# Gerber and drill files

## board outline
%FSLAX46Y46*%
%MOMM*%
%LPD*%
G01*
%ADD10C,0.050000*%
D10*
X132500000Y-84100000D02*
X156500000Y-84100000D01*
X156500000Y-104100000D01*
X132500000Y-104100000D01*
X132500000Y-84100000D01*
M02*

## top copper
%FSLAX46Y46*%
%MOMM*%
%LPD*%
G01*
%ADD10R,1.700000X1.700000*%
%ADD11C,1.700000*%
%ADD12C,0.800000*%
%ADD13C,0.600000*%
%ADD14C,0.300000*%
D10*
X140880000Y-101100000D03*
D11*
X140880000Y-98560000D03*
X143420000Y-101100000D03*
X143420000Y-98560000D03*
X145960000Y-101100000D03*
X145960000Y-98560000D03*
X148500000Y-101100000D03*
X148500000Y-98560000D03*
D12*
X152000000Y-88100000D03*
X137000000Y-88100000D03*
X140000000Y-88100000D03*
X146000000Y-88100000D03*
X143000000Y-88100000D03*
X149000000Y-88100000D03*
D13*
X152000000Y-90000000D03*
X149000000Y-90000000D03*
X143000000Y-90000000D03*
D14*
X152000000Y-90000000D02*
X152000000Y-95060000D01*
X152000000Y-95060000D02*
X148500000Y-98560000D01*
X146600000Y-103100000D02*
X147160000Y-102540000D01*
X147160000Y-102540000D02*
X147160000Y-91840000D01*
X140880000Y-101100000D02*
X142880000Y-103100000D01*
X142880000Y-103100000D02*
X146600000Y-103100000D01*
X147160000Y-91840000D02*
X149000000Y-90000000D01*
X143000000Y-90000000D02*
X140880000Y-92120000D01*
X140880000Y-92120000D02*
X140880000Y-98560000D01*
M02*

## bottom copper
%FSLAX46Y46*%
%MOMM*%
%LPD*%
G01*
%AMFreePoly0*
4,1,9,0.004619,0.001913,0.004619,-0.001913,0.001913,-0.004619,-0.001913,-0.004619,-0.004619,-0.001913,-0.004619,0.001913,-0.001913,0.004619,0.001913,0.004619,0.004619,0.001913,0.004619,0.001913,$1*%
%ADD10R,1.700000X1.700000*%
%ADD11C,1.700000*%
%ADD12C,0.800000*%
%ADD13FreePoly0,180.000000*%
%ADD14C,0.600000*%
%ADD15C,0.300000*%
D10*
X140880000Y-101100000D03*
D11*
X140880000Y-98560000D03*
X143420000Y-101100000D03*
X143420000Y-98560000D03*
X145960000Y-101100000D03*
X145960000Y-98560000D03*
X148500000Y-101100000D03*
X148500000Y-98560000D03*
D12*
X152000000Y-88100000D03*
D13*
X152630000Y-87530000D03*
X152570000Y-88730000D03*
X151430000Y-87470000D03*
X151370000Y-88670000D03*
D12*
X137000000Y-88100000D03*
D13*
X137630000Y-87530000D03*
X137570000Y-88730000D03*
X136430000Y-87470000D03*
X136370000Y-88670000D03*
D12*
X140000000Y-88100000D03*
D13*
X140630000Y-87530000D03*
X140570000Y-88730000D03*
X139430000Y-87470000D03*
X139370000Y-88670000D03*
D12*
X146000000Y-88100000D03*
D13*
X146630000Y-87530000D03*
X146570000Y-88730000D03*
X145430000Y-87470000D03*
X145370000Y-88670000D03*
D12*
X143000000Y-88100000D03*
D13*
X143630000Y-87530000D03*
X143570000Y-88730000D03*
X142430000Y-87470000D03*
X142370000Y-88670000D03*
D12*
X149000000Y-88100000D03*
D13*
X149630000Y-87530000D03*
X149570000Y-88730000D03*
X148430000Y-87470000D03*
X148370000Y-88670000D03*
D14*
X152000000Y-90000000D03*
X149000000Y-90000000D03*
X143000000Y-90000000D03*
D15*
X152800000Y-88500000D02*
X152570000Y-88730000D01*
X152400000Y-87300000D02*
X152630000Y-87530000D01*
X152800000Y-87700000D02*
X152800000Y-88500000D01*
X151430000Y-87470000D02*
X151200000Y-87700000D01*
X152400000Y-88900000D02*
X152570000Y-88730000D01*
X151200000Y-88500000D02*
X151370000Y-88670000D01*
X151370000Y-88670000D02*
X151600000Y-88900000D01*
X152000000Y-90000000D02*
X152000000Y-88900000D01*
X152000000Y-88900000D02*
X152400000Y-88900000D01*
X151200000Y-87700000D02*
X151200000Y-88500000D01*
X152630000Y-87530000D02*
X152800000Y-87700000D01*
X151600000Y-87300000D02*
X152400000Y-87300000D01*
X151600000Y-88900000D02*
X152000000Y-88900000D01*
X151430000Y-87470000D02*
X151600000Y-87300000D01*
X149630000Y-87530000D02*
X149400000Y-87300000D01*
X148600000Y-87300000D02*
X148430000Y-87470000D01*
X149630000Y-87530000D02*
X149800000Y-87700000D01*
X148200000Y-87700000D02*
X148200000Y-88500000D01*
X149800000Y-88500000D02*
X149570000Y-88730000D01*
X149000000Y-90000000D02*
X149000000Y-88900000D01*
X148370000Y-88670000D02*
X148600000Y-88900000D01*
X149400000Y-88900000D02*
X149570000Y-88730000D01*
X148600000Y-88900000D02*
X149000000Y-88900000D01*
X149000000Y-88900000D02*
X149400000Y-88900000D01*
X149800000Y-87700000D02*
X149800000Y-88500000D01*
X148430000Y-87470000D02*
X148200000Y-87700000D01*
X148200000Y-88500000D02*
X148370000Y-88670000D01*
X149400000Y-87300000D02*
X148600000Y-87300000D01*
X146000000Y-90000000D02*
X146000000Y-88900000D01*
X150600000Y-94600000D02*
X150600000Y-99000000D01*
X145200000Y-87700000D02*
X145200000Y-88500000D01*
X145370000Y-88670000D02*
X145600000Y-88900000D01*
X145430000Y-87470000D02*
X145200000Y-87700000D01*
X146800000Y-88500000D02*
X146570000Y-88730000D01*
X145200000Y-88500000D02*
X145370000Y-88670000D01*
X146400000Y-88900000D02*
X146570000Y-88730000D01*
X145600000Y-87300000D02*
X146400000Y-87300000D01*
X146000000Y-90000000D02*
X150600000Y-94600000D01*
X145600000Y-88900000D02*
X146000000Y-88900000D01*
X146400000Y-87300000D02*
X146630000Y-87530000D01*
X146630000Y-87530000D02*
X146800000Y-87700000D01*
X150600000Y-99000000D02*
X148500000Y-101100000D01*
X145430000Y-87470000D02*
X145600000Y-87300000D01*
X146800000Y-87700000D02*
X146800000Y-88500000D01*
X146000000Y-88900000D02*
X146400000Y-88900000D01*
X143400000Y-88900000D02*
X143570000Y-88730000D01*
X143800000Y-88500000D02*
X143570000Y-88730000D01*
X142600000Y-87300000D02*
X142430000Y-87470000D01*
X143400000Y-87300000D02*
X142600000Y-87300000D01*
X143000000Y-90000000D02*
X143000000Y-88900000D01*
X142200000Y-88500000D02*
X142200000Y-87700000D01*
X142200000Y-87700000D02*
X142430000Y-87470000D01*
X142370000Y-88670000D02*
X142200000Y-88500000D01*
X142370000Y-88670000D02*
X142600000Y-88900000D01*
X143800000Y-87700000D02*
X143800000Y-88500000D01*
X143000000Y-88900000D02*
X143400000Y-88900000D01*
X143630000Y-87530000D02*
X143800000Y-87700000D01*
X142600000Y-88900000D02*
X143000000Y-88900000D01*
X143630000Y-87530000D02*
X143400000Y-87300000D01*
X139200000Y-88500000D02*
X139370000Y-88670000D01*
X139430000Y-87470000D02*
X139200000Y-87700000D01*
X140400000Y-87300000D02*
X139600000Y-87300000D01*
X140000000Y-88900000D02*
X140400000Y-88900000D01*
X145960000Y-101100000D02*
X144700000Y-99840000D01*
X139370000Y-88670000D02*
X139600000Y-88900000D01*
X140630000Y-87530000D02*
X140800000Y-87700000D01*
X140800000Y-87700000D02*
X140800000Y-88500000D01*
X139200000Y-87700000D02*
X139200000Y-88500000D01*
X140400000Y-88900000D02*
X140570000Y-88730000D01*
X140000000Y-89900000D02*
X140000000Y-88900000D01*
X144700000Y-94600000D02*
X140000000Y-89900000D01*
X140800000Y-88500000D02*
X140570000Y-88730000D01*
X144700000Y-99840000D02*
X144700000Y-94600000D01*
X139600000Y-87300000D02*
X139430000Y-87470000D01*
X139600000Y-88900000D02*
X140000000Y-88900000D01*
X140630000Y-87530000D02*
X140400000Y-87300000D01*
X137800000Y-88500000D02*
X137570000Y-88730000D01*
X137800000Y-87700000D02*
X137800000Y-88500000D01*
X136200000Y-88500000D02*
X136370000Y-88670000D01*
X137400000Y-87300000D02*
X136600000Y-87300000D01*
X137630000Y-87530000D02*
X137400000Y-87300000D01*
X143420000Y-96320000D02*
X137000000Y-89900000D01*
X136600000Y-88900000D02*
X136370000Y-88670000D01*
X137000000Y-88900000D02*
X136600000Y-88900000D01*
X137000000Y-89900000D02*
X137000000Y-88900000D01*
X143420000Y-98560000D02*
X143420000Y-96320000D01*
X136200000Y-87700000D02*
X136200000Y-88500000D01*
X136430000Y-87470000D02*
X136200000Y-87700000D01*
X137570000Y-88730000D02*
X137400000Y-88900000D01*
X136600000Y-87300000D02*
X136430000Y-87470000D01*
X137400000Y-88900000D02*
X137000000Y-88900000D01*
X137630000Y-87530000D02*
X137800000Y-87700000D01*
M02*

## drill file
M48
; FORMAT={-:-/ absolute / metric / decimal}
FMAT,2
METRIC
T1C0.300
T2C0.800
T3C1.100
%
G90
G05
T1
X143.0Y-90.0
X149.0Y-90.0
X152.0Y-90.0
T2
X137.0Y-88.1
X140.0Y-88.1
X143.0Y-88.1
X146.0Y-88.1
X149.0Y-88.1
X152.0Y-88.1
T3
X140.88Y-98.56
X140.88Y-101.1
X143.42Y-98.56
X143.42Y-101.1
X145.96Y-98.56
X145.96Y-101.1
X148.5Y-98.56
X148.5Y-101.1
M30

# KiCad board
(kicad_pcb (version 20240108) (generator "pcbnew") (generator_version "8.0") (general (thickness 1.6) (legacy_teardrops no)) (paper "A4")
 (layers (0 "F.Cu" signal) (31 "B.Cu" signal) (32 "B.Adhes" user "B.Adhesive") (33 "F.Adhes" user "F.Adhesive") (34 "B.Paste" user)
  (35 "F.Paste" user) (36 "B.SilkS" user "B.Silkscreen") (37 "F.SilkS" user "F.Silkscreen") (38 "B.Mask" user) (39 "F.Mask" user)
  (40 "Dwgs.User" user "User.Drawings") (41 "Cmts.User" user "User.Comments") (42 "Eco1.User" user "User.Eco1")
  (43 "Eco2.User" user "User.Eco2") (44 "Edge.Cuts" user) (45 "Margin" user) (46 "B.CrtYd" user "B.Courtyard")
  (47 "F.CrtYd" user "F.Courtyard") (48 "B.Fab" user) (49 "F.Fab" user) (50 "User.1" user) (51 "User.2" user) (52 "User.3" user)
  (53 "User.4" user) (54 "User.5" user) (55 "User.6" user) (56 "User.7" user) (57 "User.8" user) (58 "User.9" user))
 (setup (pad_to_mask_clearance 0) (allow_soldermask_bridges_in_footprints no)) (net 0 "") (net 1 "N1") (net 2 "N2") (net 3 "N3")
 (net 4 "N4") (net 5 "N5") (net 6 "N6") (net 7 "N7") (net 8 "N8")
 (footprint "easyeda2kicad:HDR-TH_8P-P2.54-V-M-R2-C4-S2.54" (layer "F.Cu") (at 144.69 99.83)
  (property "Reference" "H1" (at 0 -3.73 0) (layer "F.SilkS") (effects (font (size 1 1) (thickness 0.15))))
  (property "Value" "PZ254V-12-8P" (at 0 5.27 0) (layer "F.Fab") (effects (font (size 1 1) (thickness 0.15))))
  (pad "1" thru_hole rect (at -3.81 1.27) (size 1.7 1.7) (drill 1.099998) (layers "*.Cu" "*.Mask") (remove_unused_layers no) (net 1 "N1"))
  (pad "2" thru_hole circle (at -3.81 -1.27) (size 1.7 1.7) (drill 1.099998) (layers "*.Cu" "*.Mask") (remove_unused_layers no) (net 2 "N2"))
  (pad "3" thru_hole circle (at -1.27 1.27) (size 1.7 1.7) (drill 1.099998) (layers "*.Cu" "*.Mask") (remove_unused_layers no) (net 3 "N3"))
  (pad "4" thru_hole circle (at -1.27 -1.27) (size 1.7 1.7) (drill 1.099998) (layers "*.Cu" "*.Mask") (remove_unused_layers no) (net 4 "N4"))
  (pad "5" thru_hole circle (at 1.27 1.27) (size 1.7 1.7) (drill 1.099998) (layers "*.Cu" "*.Mask") (remove_unused_layers no) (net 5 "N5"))
  (pad "6" thru_hole circle (at 1.27 -1.27) (size 1.7 1.7) (drill 1.099998) (layers "*.Cu" "*.Mask") (remove_unused_layers no) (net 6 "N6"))
  (pad "7" thru_hole circle (at 3.81 1.27) (size 1.7 1.7) (drill 1.099998) (layers "*.Cu" "*.Mask") (remove_unused_layers no) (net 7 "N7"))
  (pad "8" thru_hole circle (at 3.81 -1.27) (size 1.7 1.7) (drill 1.099998) (layers "*.Cu" "*.Mask") (remove_unused_layers no) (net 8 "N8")))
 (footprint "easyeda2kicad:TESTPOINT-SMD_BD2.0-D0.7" (layer "B.Cu") (at 152 88.1 180)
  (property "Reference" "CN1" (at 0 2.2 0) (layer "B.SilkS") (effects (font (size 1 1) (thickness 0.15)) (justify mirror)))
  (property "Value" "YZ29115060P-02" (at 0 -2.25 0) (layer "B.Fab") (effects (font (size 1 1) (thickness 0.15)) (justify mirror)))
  (pad "" thru_hole circle (at 0 0 180) (size 0.8 0.8) (drill 0.8) (layers "*.Cu" "*.Mask") (remove_unused_layers no))
  (pad "1" smd custom (at -0.63 0.57 180) (size 0.01 0.01) (layers "B.Cu" "B.Paste" "B.Mask") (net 8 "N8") (thermal_bridge_angle 90)
   (options (clearance outline) (anchor circle)) (primitives))
  (pad "1" smd custom (at -0.57 -0.63 180) (size 0.01 0.01) (layers "B.Cu" "B.Paste" "B.Mask") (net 8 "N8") (thermal_bridge_angle 90)
   (options (clearance outline) (anchor circle)) (primitives))
  (pad "1" smd custom (at 0.57 0.63 180) (size 0.01 0.01) (layers "B.Cu" "B.Paste" "B.Mask") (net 8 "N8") (thermal_bridge_angle 90)
   (options (clearance outline) (anchor circle)) (primitives))
  (pad "1" smd custom (at 0.63 -0.57 180) (size 0.01 0.01) (layers "B.Cu" "B.Paste" "B.Mask") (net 8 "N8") (thermal_bridge_angle 90)
   (options (clearance outline) (anchor circle)) (primitives)))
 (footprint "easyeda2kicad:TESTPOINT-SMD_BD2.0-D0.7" (layer "B.Cu") (at 137 88.1 180)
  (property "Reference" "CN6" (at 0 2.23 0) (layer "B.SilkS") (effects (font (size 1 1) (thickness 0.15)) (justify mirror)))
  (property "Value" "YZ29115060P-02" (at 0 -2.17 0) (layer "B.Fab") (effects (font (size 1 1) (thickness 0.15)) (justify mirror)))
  (pad "" thru_hole circle (at 0 0 180) (size 0.8 0.8) (drill 0.8) (layers "*.Cu" "*.Mask") (remove_unused_layers no))
  (pad "1" smd custom (at -0.63 0.57 180) (size 0.01 0.01) (layers "B.Cu" "B.Paste" "B.Mask") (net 4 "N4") (thermal_bridge_angle 90)
   (options (clearance outline) (anchor circle)) (primitives))
  (pad "1" smd custom (at -0.57 -0.63 180) (size 0.01 0.01) (layers "B.Cu" "B.Paste" "B.Mask") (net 4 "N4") (thermal_bridge_angle 90)
   (options (clearance outline) (anchor circle)) (primitives))
  (pad "1" smd custom (at 0.57 0.63 180) (size 0.01 0.01) (layers "B.Cu" "B.Paste" "B.Mask") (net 4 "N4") (thermal_bridge_angle 90)
   (options (clearance outline) (anchor circle)) (primitives))
  (pad "1" smd custom (at 0.63 -0.57 180) (size 0.01 0.01) (layers "B.Cu" "B.Paste" "B.Mask") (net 4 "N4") (thermal_bridge_angle 90)
   (options (clearance outline) (anchor circle)) (primitives)))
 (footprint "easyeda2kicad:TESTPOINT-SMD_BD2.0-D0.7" (layer "B.Cu") (at 140 88.1 180)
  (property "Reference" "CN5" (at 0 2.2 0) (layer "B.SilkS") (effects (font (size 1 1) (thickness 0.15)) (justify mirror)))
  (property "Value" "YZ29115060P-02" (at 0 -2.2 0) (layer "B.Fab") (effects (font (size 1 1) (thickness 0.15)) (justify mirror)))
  (pad "" thru_hole circle (at 0 0 180) (size 0.8 0.8) (drill 0.8) (layers "*.Cu" "*.Mask") (remove_unused_layers no))
  (pad "1" smd custom (at -0.63 0.57 180) (size 0.01 0.01) (layers "B.Cu" "B.Paste" "B.Mask") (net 5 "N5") (thermal_bridge_angle 90)
   (options (clearance outline) (anchor circle)) (primitives))
  (pad "1" smd custom (at -0.57 -0.63 180) (size 0.01 0.01) (layers "B.Cu" "B.Paste" "B.Mask") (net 5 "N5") (thermal_bridge_angle 90)
   (options (clearance outline) (anchor circle)) (primitives))
  (pad "1" smd custom (at 0.57 0.63 180) (size 0.01 0.01) (layers "B.Cu" "B.Paste" "B.Mask") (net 5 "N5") (thermal_bridge_angle 90)
   (options (clearance outline) (anchor circle)) (primitives))
  (pad "1" smd custom (at 0.63 -0.57 180) (size 0.01 0.01) (layers "B.Cu" "B.Paste" "B.Mask") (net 5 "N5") (thermal_bridge_angle 90)
   (options (clearance outline) (anchor circle)) (primitives)))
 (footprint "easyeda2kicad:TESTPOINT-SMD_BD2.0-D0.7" (layer "B.Cu") (at 146 88.1 180)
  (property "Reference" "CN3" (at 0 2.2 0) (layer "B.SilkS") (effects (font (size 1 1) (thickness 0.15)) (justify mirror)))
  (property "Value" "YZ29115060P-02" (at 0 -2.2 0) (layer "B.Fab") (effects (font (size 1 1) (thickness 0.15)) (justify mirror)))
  (pad "" thru_hole circle (at 0 0 180) (size 0.8 0.8) (drill 0.8) (layers "*.Cu" "*.Mask") (remove_unused_layers no))
  (pad "1" smd custom (at -0.63 0.57 180) (size 0.01 0.01) (layers "B.Cu" "B.Paste" "B.Mask") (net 7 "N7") (thermal_bridge_angle 90)
   (options (clearance outline) (anchor circle)) (primitives))
  (pad "1" smd custom (at -0.57 -0.63 180) (size 0.01 0.01) (layers "B.Cu" "B.Paste" "B.Mask") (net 7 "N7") (thermal_bridge_angle 90)
   (options (clearance outline) (anchor circle)) (primitives))
  (pad "1" smd custom (at 0.57 0.63 180) (size 0.01 0.01) (layers "B.Cu" "B.Paste" "B.Mask") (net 7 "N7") (thermal_bridge_angle 90)
   (options (clearance outline) (anchor circle)) (primitives))
  (pad "1" smd custom (at 0.63 -0.57 180) (size 0.01 0.01) (layers "B.Cu" "B.Paste" "B.Mask") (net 7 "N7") (thermal_bridge_angle 90)
   (options (clearance outline) (anchor circle)) (primitives)))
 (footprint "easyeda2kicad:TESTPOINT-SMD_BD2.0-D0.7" (layer "B.Cu") (at 143 88.1 180)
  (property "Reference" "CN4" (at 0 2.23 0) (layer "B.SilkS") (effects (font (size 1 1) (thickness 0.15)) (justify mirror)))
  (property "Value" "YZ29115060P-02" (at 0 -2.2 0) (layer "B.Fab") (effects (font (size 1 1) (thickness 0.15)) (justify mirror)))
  (pad "" thru_hole circle (at 0 0 180) (size 0.8 0.8) (drill 0.8) (layers "*.Cu" "*.Mask") (remove_unused_layers no))
  (pad "1" smd custom (at -0.63 0.57 180) (size 0.01 0.01) (layers "B.Cu" "B.Paste" "B.Mask") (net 2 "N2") (thermal_bridge_angle 90)
   (options (clearance outline) (anchor circle)) (primitives))
  (pad "1" smd custom (at -0.57 -0.63 180) (size 0.01 0.01) (layers "B.Cu" "B.Paste" "B.Mask") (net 2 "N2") (thermal_bridge_angle 90)
   (options (clearance outline) (anchor circle)) (primitives))
  (pad "1" smd custom (at 0.57 0.63 180) (size 0.01 0.01) (layers "B.Cu" "B.Paste" "B.Mask") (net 2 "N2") (thermal_bridge_angle 90)
   (options (clearance outline) (anchor circle)) (primitives))
  (pad "1" smd custom (at 0.63 -0.57 180) (size 0.01 0.01) (layers "B.Cu" "B.Paste" "B.Mask") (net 2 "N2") (thermal_bridge_angle 90)
   (options (clearance outline) (anchor circle)) (primitives)))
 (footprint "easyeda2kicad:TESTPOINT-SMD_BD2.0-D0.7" (layer "B.Cu") (at 149 88.1 180)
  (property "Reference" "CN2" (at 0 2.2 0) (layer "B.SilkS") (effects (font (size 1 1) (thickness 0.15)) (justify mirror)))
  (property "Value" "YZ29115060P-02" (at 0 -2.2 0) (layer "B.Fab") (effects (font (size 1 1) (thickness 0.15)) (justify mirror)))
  (pad "" thru_hole circle (at 0 0 180) (size 0.8 0.8) (drill 0.8) (layers "*.Cu" "*.Mask") (remove_unused_layers no))
  (pad "1" smd custom (at -0.63 0.57 180) (size 0.01 0.01) (layers "B.Cu" "B.Paste" "B.Mask") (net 1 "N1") (thermal_bridge_angle 90)
   (options (clearance outline) (anchor circle)) (primitives))
  (pad "1" smd custom (at -0.57 -0.63 180) (size 0.01 0.01) (layers "B.Cu" "B.Paste" "B.Mask") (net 1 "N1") (thermal_bridge_angle 90)
   (options (clearance outline) (anchor circle)) (primitives))
  (pad "1" smd custom (at 0.57 0.63 180) (size 0.01 0.01) (layers "B.Cu" "B.Paste" "B.Mask") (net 1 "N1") (thermal_bridge_angle 90)
   (options (clearance outline) (anchor circle)) (primitives))
  (pad "1" smd custom (at 0.63 -0.57 180) (size 0.01 0.01) (layers "B.Cu" "B.Paste" "B.Mask") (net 1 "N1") (thermal_bridge_angle 90)
   (options (clearance outline) (anchor circle)) (primitives)))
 (gr_rect (start 132.5 84.1) (end 156.5 104.1) (stroke (width 0.05) (type default)) (fill none) (layer "Edge.Cuts"))
 (segment (start 152 90) (end 152 95.06) (width 0.3) (layer "F.Cu") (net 8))
 (segment (start 152 95.06) (end 148.5 98.56) (width 0.3) (layer "F.Cu") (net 8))
 (via (at 152 90) (size 0.6) (drill 0.3) (layers "F.Cu" "B.Cu") (free yes) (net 8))
 (segment (start 152.8 88.5) (end 152.57 88.73) (width 0.3) (layer "B.Cu") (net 8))
 (segment (start 152.4 87.3) (end 152.63 87.53) (width 0.3) (layer "B.Cu") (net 8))
 (segment (start 152.8 87.7) (end 152.8 88.5) (width 0.3) (layer "B.Cu") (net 8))
 (segment (start 151.43 87.47) (end 151.2 87.7) (width 0.3) (layer "B.Cu") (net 8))
 (segment (start 152.4 88.9) (end 152.57 88.73) (width 0.3) (layer "B.Cu") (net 8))
 (segment (start 151.2 88.5) (end 151.37 88.67) (width 0.3) (layer "B.Cu") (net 8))
 (segment (start 151.37 88.67) (end 151.6 88.9) (width 0.3) (layer "B.Cu") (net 8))
 (segment (start 152 90) (end 152 88.9) (width 0.3) (layer "B.Cu") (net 8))
 (segment (start 152 88.9) (end 152.4 88.9) (width 0.3) (layer "B.Cu") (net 8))
 (segment (start 151.2 87.7) (end 151.2 88.5) (width 0.3) (layer "B.Cu") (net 8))
 (segment (start 152.63 87.53) (end 152.8 87.7) (width 0.3) (layer "B.Cu") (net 8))
 (segment (start 151.6 87.3) (end 152.4 87.3) (width 0.3) (layer "B.Cu") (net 8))
 (segment (start 151.6 88.9) (end 152 88.9) (width 0.3) (layer "B.Cu") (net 8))
 (segment (start 151.43 87.47) (end 151.6 87.3) (width 0.3) (layer "B.Cu") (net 8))
 (segment (start 146.6 103.1) (end 147.16 102.54) (width 0.3) (layer "F.Cu") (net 1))
 (segment (start 147.16 102.54) (end 147.16 91.84) (width 0.3) (layer "F.Cu") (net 1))
 (segment (start 140.88 101.1) (end 142.88 103.1) (width 0.3) (layer "F.Cu") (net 1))
 (segment (start 142.88 103.1) (end 146.6 103.1) (width 0.3) (layer "F.Cu") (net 1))
 (segment (start 147.16 91.84) (end 149 90) (width 0.3) (layer "F.Cu") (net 1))
 (via (at 149 90) (size 0.6) (drill 0.3) (layers "F.Cu" "B.Cu") (free yes) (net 1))
 (segment (start 149.63 87.53) (end 149.4 87.3) (width 0.3) (layer "B.Cu") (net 1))
 (segment (start 148.6 87.3) (end 148.43 87.47) (width 0.3) (layer "B.Cu") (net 1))
 (segment (start 149.63 87.53) (end 149.8 87.7) (width 0.3) (layer "B.Cu") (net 1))
 (segment (start 148.2 87.7) (end 148.2 88.5) (width 0.3) (layer "B.Cu") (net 1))
 (segment (start 149.8 88.5) (end 149.57 88.73) (width 0.3) (layer "B.Cu") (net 1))
 (segment (start 149 90) (end 149 88.9) (width 0.3) (layer "B.Cu") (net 1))
 (segment (start 148.37 88.67) (end 148.6 88.9) (width 0.3) (layer "B.Cu") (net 1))
 (segment (start 149.4 88.9) (end 149.57 88.73) (width 0.3) (layer "B.Cu") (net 1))
 (segment (start 148.6 88.9) (end 149 88.9) (width 0.3) (layer "B.Cu") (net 1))
 (segment (start 149 88.9) (end 149.4 88.9) (width 0.3) (layer "B.Cu") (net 1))
 (segment (start 149.8 87.7) (end 149.8 88.5) (width 0.3) (layer "B.Cu") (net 1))
 (segment (start 148.43 87.47) (end 148.2 87.7) (width 0.3) (layer "B.Cu") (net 1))
 (segment (start 148.2 88.5) (end 148.37 88.67) (width 0.3) (layer "B.Cu") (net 1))
 (segment (start 149.4 87.3) (end 148.6 87.3) (width 0.3) (layer "B.Cu") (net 1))
 (segment (start 146 90) (end 146 88.9) (width 0.3) (layer "B.Cu") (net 7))
 (segment (start 150.6 94.6) (end 150.6 99) (width 0.3) (layer "B.Cu") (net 7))
 (segment (start 145.2 87.7) (end 145.2 88.5) (width 0.3) (layer "B.Cu") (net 7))
 (segment (start 145.37 88.67) (end 145.6 88.9) (width 0.3) (layer "B.Cu") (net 7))
 (segment (start 145.43 87.47) (end 145.2 87.7) (width 0.3) (layer "B.Cu") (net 7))
 (segment (start 146.8 88.5) (end 146.57 88.73) (width 0.3) (layer "B.Cu") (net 7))
 (segment (start 145.2 88.5) (end 145.37 88.67) (width 0.3) (layer "B.Cu") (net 7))
 (segment (start 146.4 88.9) (end 146.57 88.73) (width 0.3) (layer "B.Cu") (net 7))
 (segment (start 145.6 87.3) (end 146.4 87.3) (width 0.3) (layer "B.Cu") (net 7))
 (segment (start 146 90) (end 150.6 94.6) (width 0.3) (layer "B.Cu") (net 7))
 (segment (start 145.6 88.9) (end 146 88.9) (width 0.3) (layer "B.Cu") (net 7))
 (segment (start 146.4 87.3) (end 146.63 87.53) (width 0.3) (layer "B.Cu") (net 7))
 (segment (start 146.63 87.53) (end 146.8 87.7) (width 0.3) (layer "B.Cu") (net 7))
 (segment (start 150.6 99) (end 148.5 101.1) (width 0.3) (layer "B.Cu") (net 7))
 (segment (start 145.43 87.47) (end 145.6 87.3) (width 0.3) (layer "B.Cu") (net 7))
 (segment (start 146.8 87.7) (end 146.8 88.5) (width 0.3) (layer "B.Cu") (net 7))
 (segment (start 146 88.9) (end 146.4 88.9) (width 0.3) (layer "B.Cu") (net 7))
 (segment (start 143 90) (end 140.88 92.12) (width 0.3) (layer "F.Cu") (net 2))
 (segment (start 140.88 92.12) (end 140.88 98.56) (width 0.3) (layer "F.Cu") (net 2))
 (via (at 143 90) (size 0.6) (drill 0.3) (layers "F.Cu" "B.Cu") (free yes) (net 2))
 (segment (start 143.4 88.9) (end 143.57 88.73) (width 0.3) (layer "B.Cu") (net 2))
 (segment (start 143.8 88.5) (end 143.57 88.73) (width 0.3) (layer "B.Cu") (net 2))
 (segment (start 142.6 87.3) (end 142.43 87.47) (width 0.3) (layer "B.Cu") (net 2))
 (segment (start 143.4 87.3) (end 142.6 87.3) (width 0.3) (layer "B.Cu") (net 2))
 (segment (start 143 90) (end 143 88.9) (width 0.3) (layer "B.Cu") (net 2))
 (segment (start 142.2 88.5) (end 142.2 87.7) (width 0.3) (layer "B.Cu") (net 2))
 (segment (start 142.2 87.7) (end 142.43 87.47) (width 0.3) (layer "B.Cu") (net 2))
 (segment (start 142.37 88.67) (end 142.2 88.5) (width 0.3) (layer "B.Cu") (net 2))
 (segment (start 142.37 88.67) (end 142.6 88.9) (width 0.3) (layer "B.Cu") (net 2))
 (segment (start 143.8 87.7) (end 143.8 88.5) (width 0.3) (layer "B.Cu") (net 2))
 (segment (start 143 88.9) (end 143.4 88.9) (width 0.3) (layer "B.Cu") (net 2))
 (segment (start 143.63 87.53) (end 143.8 87.7) (width 0.3) (layer "B.Cu") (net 2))
 (segment (start 142.6 88.9) (end 143 88.9) (width 0.3) (layer "B.Cu") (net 2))
 (segment (start 143.63 87.53) (end 143.4 87.3) (width 0.3) (layer "B.Cu") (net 2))
 (segment (start 139.2 88.5) (end 139.37 88.67) (width 0.3) (layer "B.Cu") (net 5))
 (segment (start 139.43 87.47) (end 139.2 87.7) (width 0.3) (layer "B.Cu") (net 5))
 (segment (start 140.4 87.3) (end 139.6 87.3) (width 0.3) (layer "B.Cu") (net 5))
 (segment (start 140 88.9) (end 140.4 88.9) (width 0.3) (layer "B.Cu") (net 5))
 (segment (start 145.96 101.1) (end 144.7 99.84) (width 0.3) (layer "B.Cu") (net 5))
 (segment (start 139.37 88.67) (end 139.6 88.9) (width 0.3) (layer "B.Cu") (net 5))
 (segment (start 140.63 87.53) (end 140.8 87.7) (width 0.3) (layer "B.Cu") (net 5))
 (segment (start 140.8 87.7) (end 140.8 88.5) (width 0.3) (layer "B.Cu") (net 5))
 (segment (start 139.2 87.7) (end 139.2 88.5) (width 0.3) (layer "B.Cu") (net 5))
 (segment (start 140.4 88.9) (end 140.57 88.73) (width 0.3) (layer "B.Cu") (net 5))
 (segment (start 140 89.9) (end 140 88.9) (width 0.3) (layer "B.Cu") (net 5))
 (segment (start 144.7 94.6) (end 140 89.9) (width 0.3) (layer "B.Cu") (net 5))
 (segment (start 140.8 88.5) (end 140.57 88.73) (width 0.3) (layer "B.Cu") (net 5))
 (segment (start 144.7 99.84) (end 144.7 94.6) (width 0.3) (layer "B.Cu") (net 5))
 (segment (start 139.6 87.3) (end 139.43 87.47) (width 0.3) (layer "B.Cu") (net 5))
 (segment (start 139.6 88.9) (end 140 88.9) (width 0.3) (layer "B.Cu") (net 5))
 (segment (start 140.63 87.53) (end 140.4 87.3) (width 0.3) (layer "B.Cu") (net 5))
 (segment (start 137.8 88.5) (end 137.57 88.73) (width 0.3) (layer "B.Cu") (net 4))
 (segment (start 137.8 87.7) (end 137.8 88.5) (width 0.3) (layer "B.Cu") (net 4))
 (segment (start 136.2 88.5) (end 136.37 88.67) (width 0.3) (layer "B.Cu") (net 4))
 (segment (start 137.4 87.3) (end 136.6 87.3) (width 0.3) (layer "B.Cu") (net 4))
 (segment (start 137.63 87.53) (end 137.4 87.3) (width 0.3) (layer "B.Cu") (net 4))
 (segment (start 143.42 96.32) (end 137 89.9) (width 0.3) (layer "B.Cu") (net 4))
 (segment (start 136.6 88.9) (end 136.37 88.67) (width 0.3) (layer "B.Cu") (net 4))
 (segment (start 137 88.9) (end 136.6 88.9) (width 0.3) (layer "B.Cu") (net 4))
 (segment (start 137 89.9) (end 137 88.9) (width 0.3) (layer "B.Cu") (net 4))
 (segment (start 143.42 98.56) (end 143.42 96.32) (width 0.3) (layer "B.Cu") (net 4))
 (segment (start 136.2 87.7) (end 136.2 88.5) (width 0.3) (layer "B.Cu") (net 4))
 (segment (start 136.43 87.47) (end 136.2 87.7) (width 0.3) (layer "B.Cu") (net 4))
 (segment (start 137.57 88.73) (end 137.4 88.9) (width 0.3) (layer "B.Cu") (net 4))
 (segment (start 136.6 87.3) (end 136.43 87.47) (width 0.3) (layer "B.Cu") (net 4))
 (segment (start 137.4 88.9) (end 137 88.9) (width 0.3) (layer "B.Cu") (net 4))
 (segment (start 137.63 87.53) (end 137.8 87.7) (width 0.3) (layer "B.Cu") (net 4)))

